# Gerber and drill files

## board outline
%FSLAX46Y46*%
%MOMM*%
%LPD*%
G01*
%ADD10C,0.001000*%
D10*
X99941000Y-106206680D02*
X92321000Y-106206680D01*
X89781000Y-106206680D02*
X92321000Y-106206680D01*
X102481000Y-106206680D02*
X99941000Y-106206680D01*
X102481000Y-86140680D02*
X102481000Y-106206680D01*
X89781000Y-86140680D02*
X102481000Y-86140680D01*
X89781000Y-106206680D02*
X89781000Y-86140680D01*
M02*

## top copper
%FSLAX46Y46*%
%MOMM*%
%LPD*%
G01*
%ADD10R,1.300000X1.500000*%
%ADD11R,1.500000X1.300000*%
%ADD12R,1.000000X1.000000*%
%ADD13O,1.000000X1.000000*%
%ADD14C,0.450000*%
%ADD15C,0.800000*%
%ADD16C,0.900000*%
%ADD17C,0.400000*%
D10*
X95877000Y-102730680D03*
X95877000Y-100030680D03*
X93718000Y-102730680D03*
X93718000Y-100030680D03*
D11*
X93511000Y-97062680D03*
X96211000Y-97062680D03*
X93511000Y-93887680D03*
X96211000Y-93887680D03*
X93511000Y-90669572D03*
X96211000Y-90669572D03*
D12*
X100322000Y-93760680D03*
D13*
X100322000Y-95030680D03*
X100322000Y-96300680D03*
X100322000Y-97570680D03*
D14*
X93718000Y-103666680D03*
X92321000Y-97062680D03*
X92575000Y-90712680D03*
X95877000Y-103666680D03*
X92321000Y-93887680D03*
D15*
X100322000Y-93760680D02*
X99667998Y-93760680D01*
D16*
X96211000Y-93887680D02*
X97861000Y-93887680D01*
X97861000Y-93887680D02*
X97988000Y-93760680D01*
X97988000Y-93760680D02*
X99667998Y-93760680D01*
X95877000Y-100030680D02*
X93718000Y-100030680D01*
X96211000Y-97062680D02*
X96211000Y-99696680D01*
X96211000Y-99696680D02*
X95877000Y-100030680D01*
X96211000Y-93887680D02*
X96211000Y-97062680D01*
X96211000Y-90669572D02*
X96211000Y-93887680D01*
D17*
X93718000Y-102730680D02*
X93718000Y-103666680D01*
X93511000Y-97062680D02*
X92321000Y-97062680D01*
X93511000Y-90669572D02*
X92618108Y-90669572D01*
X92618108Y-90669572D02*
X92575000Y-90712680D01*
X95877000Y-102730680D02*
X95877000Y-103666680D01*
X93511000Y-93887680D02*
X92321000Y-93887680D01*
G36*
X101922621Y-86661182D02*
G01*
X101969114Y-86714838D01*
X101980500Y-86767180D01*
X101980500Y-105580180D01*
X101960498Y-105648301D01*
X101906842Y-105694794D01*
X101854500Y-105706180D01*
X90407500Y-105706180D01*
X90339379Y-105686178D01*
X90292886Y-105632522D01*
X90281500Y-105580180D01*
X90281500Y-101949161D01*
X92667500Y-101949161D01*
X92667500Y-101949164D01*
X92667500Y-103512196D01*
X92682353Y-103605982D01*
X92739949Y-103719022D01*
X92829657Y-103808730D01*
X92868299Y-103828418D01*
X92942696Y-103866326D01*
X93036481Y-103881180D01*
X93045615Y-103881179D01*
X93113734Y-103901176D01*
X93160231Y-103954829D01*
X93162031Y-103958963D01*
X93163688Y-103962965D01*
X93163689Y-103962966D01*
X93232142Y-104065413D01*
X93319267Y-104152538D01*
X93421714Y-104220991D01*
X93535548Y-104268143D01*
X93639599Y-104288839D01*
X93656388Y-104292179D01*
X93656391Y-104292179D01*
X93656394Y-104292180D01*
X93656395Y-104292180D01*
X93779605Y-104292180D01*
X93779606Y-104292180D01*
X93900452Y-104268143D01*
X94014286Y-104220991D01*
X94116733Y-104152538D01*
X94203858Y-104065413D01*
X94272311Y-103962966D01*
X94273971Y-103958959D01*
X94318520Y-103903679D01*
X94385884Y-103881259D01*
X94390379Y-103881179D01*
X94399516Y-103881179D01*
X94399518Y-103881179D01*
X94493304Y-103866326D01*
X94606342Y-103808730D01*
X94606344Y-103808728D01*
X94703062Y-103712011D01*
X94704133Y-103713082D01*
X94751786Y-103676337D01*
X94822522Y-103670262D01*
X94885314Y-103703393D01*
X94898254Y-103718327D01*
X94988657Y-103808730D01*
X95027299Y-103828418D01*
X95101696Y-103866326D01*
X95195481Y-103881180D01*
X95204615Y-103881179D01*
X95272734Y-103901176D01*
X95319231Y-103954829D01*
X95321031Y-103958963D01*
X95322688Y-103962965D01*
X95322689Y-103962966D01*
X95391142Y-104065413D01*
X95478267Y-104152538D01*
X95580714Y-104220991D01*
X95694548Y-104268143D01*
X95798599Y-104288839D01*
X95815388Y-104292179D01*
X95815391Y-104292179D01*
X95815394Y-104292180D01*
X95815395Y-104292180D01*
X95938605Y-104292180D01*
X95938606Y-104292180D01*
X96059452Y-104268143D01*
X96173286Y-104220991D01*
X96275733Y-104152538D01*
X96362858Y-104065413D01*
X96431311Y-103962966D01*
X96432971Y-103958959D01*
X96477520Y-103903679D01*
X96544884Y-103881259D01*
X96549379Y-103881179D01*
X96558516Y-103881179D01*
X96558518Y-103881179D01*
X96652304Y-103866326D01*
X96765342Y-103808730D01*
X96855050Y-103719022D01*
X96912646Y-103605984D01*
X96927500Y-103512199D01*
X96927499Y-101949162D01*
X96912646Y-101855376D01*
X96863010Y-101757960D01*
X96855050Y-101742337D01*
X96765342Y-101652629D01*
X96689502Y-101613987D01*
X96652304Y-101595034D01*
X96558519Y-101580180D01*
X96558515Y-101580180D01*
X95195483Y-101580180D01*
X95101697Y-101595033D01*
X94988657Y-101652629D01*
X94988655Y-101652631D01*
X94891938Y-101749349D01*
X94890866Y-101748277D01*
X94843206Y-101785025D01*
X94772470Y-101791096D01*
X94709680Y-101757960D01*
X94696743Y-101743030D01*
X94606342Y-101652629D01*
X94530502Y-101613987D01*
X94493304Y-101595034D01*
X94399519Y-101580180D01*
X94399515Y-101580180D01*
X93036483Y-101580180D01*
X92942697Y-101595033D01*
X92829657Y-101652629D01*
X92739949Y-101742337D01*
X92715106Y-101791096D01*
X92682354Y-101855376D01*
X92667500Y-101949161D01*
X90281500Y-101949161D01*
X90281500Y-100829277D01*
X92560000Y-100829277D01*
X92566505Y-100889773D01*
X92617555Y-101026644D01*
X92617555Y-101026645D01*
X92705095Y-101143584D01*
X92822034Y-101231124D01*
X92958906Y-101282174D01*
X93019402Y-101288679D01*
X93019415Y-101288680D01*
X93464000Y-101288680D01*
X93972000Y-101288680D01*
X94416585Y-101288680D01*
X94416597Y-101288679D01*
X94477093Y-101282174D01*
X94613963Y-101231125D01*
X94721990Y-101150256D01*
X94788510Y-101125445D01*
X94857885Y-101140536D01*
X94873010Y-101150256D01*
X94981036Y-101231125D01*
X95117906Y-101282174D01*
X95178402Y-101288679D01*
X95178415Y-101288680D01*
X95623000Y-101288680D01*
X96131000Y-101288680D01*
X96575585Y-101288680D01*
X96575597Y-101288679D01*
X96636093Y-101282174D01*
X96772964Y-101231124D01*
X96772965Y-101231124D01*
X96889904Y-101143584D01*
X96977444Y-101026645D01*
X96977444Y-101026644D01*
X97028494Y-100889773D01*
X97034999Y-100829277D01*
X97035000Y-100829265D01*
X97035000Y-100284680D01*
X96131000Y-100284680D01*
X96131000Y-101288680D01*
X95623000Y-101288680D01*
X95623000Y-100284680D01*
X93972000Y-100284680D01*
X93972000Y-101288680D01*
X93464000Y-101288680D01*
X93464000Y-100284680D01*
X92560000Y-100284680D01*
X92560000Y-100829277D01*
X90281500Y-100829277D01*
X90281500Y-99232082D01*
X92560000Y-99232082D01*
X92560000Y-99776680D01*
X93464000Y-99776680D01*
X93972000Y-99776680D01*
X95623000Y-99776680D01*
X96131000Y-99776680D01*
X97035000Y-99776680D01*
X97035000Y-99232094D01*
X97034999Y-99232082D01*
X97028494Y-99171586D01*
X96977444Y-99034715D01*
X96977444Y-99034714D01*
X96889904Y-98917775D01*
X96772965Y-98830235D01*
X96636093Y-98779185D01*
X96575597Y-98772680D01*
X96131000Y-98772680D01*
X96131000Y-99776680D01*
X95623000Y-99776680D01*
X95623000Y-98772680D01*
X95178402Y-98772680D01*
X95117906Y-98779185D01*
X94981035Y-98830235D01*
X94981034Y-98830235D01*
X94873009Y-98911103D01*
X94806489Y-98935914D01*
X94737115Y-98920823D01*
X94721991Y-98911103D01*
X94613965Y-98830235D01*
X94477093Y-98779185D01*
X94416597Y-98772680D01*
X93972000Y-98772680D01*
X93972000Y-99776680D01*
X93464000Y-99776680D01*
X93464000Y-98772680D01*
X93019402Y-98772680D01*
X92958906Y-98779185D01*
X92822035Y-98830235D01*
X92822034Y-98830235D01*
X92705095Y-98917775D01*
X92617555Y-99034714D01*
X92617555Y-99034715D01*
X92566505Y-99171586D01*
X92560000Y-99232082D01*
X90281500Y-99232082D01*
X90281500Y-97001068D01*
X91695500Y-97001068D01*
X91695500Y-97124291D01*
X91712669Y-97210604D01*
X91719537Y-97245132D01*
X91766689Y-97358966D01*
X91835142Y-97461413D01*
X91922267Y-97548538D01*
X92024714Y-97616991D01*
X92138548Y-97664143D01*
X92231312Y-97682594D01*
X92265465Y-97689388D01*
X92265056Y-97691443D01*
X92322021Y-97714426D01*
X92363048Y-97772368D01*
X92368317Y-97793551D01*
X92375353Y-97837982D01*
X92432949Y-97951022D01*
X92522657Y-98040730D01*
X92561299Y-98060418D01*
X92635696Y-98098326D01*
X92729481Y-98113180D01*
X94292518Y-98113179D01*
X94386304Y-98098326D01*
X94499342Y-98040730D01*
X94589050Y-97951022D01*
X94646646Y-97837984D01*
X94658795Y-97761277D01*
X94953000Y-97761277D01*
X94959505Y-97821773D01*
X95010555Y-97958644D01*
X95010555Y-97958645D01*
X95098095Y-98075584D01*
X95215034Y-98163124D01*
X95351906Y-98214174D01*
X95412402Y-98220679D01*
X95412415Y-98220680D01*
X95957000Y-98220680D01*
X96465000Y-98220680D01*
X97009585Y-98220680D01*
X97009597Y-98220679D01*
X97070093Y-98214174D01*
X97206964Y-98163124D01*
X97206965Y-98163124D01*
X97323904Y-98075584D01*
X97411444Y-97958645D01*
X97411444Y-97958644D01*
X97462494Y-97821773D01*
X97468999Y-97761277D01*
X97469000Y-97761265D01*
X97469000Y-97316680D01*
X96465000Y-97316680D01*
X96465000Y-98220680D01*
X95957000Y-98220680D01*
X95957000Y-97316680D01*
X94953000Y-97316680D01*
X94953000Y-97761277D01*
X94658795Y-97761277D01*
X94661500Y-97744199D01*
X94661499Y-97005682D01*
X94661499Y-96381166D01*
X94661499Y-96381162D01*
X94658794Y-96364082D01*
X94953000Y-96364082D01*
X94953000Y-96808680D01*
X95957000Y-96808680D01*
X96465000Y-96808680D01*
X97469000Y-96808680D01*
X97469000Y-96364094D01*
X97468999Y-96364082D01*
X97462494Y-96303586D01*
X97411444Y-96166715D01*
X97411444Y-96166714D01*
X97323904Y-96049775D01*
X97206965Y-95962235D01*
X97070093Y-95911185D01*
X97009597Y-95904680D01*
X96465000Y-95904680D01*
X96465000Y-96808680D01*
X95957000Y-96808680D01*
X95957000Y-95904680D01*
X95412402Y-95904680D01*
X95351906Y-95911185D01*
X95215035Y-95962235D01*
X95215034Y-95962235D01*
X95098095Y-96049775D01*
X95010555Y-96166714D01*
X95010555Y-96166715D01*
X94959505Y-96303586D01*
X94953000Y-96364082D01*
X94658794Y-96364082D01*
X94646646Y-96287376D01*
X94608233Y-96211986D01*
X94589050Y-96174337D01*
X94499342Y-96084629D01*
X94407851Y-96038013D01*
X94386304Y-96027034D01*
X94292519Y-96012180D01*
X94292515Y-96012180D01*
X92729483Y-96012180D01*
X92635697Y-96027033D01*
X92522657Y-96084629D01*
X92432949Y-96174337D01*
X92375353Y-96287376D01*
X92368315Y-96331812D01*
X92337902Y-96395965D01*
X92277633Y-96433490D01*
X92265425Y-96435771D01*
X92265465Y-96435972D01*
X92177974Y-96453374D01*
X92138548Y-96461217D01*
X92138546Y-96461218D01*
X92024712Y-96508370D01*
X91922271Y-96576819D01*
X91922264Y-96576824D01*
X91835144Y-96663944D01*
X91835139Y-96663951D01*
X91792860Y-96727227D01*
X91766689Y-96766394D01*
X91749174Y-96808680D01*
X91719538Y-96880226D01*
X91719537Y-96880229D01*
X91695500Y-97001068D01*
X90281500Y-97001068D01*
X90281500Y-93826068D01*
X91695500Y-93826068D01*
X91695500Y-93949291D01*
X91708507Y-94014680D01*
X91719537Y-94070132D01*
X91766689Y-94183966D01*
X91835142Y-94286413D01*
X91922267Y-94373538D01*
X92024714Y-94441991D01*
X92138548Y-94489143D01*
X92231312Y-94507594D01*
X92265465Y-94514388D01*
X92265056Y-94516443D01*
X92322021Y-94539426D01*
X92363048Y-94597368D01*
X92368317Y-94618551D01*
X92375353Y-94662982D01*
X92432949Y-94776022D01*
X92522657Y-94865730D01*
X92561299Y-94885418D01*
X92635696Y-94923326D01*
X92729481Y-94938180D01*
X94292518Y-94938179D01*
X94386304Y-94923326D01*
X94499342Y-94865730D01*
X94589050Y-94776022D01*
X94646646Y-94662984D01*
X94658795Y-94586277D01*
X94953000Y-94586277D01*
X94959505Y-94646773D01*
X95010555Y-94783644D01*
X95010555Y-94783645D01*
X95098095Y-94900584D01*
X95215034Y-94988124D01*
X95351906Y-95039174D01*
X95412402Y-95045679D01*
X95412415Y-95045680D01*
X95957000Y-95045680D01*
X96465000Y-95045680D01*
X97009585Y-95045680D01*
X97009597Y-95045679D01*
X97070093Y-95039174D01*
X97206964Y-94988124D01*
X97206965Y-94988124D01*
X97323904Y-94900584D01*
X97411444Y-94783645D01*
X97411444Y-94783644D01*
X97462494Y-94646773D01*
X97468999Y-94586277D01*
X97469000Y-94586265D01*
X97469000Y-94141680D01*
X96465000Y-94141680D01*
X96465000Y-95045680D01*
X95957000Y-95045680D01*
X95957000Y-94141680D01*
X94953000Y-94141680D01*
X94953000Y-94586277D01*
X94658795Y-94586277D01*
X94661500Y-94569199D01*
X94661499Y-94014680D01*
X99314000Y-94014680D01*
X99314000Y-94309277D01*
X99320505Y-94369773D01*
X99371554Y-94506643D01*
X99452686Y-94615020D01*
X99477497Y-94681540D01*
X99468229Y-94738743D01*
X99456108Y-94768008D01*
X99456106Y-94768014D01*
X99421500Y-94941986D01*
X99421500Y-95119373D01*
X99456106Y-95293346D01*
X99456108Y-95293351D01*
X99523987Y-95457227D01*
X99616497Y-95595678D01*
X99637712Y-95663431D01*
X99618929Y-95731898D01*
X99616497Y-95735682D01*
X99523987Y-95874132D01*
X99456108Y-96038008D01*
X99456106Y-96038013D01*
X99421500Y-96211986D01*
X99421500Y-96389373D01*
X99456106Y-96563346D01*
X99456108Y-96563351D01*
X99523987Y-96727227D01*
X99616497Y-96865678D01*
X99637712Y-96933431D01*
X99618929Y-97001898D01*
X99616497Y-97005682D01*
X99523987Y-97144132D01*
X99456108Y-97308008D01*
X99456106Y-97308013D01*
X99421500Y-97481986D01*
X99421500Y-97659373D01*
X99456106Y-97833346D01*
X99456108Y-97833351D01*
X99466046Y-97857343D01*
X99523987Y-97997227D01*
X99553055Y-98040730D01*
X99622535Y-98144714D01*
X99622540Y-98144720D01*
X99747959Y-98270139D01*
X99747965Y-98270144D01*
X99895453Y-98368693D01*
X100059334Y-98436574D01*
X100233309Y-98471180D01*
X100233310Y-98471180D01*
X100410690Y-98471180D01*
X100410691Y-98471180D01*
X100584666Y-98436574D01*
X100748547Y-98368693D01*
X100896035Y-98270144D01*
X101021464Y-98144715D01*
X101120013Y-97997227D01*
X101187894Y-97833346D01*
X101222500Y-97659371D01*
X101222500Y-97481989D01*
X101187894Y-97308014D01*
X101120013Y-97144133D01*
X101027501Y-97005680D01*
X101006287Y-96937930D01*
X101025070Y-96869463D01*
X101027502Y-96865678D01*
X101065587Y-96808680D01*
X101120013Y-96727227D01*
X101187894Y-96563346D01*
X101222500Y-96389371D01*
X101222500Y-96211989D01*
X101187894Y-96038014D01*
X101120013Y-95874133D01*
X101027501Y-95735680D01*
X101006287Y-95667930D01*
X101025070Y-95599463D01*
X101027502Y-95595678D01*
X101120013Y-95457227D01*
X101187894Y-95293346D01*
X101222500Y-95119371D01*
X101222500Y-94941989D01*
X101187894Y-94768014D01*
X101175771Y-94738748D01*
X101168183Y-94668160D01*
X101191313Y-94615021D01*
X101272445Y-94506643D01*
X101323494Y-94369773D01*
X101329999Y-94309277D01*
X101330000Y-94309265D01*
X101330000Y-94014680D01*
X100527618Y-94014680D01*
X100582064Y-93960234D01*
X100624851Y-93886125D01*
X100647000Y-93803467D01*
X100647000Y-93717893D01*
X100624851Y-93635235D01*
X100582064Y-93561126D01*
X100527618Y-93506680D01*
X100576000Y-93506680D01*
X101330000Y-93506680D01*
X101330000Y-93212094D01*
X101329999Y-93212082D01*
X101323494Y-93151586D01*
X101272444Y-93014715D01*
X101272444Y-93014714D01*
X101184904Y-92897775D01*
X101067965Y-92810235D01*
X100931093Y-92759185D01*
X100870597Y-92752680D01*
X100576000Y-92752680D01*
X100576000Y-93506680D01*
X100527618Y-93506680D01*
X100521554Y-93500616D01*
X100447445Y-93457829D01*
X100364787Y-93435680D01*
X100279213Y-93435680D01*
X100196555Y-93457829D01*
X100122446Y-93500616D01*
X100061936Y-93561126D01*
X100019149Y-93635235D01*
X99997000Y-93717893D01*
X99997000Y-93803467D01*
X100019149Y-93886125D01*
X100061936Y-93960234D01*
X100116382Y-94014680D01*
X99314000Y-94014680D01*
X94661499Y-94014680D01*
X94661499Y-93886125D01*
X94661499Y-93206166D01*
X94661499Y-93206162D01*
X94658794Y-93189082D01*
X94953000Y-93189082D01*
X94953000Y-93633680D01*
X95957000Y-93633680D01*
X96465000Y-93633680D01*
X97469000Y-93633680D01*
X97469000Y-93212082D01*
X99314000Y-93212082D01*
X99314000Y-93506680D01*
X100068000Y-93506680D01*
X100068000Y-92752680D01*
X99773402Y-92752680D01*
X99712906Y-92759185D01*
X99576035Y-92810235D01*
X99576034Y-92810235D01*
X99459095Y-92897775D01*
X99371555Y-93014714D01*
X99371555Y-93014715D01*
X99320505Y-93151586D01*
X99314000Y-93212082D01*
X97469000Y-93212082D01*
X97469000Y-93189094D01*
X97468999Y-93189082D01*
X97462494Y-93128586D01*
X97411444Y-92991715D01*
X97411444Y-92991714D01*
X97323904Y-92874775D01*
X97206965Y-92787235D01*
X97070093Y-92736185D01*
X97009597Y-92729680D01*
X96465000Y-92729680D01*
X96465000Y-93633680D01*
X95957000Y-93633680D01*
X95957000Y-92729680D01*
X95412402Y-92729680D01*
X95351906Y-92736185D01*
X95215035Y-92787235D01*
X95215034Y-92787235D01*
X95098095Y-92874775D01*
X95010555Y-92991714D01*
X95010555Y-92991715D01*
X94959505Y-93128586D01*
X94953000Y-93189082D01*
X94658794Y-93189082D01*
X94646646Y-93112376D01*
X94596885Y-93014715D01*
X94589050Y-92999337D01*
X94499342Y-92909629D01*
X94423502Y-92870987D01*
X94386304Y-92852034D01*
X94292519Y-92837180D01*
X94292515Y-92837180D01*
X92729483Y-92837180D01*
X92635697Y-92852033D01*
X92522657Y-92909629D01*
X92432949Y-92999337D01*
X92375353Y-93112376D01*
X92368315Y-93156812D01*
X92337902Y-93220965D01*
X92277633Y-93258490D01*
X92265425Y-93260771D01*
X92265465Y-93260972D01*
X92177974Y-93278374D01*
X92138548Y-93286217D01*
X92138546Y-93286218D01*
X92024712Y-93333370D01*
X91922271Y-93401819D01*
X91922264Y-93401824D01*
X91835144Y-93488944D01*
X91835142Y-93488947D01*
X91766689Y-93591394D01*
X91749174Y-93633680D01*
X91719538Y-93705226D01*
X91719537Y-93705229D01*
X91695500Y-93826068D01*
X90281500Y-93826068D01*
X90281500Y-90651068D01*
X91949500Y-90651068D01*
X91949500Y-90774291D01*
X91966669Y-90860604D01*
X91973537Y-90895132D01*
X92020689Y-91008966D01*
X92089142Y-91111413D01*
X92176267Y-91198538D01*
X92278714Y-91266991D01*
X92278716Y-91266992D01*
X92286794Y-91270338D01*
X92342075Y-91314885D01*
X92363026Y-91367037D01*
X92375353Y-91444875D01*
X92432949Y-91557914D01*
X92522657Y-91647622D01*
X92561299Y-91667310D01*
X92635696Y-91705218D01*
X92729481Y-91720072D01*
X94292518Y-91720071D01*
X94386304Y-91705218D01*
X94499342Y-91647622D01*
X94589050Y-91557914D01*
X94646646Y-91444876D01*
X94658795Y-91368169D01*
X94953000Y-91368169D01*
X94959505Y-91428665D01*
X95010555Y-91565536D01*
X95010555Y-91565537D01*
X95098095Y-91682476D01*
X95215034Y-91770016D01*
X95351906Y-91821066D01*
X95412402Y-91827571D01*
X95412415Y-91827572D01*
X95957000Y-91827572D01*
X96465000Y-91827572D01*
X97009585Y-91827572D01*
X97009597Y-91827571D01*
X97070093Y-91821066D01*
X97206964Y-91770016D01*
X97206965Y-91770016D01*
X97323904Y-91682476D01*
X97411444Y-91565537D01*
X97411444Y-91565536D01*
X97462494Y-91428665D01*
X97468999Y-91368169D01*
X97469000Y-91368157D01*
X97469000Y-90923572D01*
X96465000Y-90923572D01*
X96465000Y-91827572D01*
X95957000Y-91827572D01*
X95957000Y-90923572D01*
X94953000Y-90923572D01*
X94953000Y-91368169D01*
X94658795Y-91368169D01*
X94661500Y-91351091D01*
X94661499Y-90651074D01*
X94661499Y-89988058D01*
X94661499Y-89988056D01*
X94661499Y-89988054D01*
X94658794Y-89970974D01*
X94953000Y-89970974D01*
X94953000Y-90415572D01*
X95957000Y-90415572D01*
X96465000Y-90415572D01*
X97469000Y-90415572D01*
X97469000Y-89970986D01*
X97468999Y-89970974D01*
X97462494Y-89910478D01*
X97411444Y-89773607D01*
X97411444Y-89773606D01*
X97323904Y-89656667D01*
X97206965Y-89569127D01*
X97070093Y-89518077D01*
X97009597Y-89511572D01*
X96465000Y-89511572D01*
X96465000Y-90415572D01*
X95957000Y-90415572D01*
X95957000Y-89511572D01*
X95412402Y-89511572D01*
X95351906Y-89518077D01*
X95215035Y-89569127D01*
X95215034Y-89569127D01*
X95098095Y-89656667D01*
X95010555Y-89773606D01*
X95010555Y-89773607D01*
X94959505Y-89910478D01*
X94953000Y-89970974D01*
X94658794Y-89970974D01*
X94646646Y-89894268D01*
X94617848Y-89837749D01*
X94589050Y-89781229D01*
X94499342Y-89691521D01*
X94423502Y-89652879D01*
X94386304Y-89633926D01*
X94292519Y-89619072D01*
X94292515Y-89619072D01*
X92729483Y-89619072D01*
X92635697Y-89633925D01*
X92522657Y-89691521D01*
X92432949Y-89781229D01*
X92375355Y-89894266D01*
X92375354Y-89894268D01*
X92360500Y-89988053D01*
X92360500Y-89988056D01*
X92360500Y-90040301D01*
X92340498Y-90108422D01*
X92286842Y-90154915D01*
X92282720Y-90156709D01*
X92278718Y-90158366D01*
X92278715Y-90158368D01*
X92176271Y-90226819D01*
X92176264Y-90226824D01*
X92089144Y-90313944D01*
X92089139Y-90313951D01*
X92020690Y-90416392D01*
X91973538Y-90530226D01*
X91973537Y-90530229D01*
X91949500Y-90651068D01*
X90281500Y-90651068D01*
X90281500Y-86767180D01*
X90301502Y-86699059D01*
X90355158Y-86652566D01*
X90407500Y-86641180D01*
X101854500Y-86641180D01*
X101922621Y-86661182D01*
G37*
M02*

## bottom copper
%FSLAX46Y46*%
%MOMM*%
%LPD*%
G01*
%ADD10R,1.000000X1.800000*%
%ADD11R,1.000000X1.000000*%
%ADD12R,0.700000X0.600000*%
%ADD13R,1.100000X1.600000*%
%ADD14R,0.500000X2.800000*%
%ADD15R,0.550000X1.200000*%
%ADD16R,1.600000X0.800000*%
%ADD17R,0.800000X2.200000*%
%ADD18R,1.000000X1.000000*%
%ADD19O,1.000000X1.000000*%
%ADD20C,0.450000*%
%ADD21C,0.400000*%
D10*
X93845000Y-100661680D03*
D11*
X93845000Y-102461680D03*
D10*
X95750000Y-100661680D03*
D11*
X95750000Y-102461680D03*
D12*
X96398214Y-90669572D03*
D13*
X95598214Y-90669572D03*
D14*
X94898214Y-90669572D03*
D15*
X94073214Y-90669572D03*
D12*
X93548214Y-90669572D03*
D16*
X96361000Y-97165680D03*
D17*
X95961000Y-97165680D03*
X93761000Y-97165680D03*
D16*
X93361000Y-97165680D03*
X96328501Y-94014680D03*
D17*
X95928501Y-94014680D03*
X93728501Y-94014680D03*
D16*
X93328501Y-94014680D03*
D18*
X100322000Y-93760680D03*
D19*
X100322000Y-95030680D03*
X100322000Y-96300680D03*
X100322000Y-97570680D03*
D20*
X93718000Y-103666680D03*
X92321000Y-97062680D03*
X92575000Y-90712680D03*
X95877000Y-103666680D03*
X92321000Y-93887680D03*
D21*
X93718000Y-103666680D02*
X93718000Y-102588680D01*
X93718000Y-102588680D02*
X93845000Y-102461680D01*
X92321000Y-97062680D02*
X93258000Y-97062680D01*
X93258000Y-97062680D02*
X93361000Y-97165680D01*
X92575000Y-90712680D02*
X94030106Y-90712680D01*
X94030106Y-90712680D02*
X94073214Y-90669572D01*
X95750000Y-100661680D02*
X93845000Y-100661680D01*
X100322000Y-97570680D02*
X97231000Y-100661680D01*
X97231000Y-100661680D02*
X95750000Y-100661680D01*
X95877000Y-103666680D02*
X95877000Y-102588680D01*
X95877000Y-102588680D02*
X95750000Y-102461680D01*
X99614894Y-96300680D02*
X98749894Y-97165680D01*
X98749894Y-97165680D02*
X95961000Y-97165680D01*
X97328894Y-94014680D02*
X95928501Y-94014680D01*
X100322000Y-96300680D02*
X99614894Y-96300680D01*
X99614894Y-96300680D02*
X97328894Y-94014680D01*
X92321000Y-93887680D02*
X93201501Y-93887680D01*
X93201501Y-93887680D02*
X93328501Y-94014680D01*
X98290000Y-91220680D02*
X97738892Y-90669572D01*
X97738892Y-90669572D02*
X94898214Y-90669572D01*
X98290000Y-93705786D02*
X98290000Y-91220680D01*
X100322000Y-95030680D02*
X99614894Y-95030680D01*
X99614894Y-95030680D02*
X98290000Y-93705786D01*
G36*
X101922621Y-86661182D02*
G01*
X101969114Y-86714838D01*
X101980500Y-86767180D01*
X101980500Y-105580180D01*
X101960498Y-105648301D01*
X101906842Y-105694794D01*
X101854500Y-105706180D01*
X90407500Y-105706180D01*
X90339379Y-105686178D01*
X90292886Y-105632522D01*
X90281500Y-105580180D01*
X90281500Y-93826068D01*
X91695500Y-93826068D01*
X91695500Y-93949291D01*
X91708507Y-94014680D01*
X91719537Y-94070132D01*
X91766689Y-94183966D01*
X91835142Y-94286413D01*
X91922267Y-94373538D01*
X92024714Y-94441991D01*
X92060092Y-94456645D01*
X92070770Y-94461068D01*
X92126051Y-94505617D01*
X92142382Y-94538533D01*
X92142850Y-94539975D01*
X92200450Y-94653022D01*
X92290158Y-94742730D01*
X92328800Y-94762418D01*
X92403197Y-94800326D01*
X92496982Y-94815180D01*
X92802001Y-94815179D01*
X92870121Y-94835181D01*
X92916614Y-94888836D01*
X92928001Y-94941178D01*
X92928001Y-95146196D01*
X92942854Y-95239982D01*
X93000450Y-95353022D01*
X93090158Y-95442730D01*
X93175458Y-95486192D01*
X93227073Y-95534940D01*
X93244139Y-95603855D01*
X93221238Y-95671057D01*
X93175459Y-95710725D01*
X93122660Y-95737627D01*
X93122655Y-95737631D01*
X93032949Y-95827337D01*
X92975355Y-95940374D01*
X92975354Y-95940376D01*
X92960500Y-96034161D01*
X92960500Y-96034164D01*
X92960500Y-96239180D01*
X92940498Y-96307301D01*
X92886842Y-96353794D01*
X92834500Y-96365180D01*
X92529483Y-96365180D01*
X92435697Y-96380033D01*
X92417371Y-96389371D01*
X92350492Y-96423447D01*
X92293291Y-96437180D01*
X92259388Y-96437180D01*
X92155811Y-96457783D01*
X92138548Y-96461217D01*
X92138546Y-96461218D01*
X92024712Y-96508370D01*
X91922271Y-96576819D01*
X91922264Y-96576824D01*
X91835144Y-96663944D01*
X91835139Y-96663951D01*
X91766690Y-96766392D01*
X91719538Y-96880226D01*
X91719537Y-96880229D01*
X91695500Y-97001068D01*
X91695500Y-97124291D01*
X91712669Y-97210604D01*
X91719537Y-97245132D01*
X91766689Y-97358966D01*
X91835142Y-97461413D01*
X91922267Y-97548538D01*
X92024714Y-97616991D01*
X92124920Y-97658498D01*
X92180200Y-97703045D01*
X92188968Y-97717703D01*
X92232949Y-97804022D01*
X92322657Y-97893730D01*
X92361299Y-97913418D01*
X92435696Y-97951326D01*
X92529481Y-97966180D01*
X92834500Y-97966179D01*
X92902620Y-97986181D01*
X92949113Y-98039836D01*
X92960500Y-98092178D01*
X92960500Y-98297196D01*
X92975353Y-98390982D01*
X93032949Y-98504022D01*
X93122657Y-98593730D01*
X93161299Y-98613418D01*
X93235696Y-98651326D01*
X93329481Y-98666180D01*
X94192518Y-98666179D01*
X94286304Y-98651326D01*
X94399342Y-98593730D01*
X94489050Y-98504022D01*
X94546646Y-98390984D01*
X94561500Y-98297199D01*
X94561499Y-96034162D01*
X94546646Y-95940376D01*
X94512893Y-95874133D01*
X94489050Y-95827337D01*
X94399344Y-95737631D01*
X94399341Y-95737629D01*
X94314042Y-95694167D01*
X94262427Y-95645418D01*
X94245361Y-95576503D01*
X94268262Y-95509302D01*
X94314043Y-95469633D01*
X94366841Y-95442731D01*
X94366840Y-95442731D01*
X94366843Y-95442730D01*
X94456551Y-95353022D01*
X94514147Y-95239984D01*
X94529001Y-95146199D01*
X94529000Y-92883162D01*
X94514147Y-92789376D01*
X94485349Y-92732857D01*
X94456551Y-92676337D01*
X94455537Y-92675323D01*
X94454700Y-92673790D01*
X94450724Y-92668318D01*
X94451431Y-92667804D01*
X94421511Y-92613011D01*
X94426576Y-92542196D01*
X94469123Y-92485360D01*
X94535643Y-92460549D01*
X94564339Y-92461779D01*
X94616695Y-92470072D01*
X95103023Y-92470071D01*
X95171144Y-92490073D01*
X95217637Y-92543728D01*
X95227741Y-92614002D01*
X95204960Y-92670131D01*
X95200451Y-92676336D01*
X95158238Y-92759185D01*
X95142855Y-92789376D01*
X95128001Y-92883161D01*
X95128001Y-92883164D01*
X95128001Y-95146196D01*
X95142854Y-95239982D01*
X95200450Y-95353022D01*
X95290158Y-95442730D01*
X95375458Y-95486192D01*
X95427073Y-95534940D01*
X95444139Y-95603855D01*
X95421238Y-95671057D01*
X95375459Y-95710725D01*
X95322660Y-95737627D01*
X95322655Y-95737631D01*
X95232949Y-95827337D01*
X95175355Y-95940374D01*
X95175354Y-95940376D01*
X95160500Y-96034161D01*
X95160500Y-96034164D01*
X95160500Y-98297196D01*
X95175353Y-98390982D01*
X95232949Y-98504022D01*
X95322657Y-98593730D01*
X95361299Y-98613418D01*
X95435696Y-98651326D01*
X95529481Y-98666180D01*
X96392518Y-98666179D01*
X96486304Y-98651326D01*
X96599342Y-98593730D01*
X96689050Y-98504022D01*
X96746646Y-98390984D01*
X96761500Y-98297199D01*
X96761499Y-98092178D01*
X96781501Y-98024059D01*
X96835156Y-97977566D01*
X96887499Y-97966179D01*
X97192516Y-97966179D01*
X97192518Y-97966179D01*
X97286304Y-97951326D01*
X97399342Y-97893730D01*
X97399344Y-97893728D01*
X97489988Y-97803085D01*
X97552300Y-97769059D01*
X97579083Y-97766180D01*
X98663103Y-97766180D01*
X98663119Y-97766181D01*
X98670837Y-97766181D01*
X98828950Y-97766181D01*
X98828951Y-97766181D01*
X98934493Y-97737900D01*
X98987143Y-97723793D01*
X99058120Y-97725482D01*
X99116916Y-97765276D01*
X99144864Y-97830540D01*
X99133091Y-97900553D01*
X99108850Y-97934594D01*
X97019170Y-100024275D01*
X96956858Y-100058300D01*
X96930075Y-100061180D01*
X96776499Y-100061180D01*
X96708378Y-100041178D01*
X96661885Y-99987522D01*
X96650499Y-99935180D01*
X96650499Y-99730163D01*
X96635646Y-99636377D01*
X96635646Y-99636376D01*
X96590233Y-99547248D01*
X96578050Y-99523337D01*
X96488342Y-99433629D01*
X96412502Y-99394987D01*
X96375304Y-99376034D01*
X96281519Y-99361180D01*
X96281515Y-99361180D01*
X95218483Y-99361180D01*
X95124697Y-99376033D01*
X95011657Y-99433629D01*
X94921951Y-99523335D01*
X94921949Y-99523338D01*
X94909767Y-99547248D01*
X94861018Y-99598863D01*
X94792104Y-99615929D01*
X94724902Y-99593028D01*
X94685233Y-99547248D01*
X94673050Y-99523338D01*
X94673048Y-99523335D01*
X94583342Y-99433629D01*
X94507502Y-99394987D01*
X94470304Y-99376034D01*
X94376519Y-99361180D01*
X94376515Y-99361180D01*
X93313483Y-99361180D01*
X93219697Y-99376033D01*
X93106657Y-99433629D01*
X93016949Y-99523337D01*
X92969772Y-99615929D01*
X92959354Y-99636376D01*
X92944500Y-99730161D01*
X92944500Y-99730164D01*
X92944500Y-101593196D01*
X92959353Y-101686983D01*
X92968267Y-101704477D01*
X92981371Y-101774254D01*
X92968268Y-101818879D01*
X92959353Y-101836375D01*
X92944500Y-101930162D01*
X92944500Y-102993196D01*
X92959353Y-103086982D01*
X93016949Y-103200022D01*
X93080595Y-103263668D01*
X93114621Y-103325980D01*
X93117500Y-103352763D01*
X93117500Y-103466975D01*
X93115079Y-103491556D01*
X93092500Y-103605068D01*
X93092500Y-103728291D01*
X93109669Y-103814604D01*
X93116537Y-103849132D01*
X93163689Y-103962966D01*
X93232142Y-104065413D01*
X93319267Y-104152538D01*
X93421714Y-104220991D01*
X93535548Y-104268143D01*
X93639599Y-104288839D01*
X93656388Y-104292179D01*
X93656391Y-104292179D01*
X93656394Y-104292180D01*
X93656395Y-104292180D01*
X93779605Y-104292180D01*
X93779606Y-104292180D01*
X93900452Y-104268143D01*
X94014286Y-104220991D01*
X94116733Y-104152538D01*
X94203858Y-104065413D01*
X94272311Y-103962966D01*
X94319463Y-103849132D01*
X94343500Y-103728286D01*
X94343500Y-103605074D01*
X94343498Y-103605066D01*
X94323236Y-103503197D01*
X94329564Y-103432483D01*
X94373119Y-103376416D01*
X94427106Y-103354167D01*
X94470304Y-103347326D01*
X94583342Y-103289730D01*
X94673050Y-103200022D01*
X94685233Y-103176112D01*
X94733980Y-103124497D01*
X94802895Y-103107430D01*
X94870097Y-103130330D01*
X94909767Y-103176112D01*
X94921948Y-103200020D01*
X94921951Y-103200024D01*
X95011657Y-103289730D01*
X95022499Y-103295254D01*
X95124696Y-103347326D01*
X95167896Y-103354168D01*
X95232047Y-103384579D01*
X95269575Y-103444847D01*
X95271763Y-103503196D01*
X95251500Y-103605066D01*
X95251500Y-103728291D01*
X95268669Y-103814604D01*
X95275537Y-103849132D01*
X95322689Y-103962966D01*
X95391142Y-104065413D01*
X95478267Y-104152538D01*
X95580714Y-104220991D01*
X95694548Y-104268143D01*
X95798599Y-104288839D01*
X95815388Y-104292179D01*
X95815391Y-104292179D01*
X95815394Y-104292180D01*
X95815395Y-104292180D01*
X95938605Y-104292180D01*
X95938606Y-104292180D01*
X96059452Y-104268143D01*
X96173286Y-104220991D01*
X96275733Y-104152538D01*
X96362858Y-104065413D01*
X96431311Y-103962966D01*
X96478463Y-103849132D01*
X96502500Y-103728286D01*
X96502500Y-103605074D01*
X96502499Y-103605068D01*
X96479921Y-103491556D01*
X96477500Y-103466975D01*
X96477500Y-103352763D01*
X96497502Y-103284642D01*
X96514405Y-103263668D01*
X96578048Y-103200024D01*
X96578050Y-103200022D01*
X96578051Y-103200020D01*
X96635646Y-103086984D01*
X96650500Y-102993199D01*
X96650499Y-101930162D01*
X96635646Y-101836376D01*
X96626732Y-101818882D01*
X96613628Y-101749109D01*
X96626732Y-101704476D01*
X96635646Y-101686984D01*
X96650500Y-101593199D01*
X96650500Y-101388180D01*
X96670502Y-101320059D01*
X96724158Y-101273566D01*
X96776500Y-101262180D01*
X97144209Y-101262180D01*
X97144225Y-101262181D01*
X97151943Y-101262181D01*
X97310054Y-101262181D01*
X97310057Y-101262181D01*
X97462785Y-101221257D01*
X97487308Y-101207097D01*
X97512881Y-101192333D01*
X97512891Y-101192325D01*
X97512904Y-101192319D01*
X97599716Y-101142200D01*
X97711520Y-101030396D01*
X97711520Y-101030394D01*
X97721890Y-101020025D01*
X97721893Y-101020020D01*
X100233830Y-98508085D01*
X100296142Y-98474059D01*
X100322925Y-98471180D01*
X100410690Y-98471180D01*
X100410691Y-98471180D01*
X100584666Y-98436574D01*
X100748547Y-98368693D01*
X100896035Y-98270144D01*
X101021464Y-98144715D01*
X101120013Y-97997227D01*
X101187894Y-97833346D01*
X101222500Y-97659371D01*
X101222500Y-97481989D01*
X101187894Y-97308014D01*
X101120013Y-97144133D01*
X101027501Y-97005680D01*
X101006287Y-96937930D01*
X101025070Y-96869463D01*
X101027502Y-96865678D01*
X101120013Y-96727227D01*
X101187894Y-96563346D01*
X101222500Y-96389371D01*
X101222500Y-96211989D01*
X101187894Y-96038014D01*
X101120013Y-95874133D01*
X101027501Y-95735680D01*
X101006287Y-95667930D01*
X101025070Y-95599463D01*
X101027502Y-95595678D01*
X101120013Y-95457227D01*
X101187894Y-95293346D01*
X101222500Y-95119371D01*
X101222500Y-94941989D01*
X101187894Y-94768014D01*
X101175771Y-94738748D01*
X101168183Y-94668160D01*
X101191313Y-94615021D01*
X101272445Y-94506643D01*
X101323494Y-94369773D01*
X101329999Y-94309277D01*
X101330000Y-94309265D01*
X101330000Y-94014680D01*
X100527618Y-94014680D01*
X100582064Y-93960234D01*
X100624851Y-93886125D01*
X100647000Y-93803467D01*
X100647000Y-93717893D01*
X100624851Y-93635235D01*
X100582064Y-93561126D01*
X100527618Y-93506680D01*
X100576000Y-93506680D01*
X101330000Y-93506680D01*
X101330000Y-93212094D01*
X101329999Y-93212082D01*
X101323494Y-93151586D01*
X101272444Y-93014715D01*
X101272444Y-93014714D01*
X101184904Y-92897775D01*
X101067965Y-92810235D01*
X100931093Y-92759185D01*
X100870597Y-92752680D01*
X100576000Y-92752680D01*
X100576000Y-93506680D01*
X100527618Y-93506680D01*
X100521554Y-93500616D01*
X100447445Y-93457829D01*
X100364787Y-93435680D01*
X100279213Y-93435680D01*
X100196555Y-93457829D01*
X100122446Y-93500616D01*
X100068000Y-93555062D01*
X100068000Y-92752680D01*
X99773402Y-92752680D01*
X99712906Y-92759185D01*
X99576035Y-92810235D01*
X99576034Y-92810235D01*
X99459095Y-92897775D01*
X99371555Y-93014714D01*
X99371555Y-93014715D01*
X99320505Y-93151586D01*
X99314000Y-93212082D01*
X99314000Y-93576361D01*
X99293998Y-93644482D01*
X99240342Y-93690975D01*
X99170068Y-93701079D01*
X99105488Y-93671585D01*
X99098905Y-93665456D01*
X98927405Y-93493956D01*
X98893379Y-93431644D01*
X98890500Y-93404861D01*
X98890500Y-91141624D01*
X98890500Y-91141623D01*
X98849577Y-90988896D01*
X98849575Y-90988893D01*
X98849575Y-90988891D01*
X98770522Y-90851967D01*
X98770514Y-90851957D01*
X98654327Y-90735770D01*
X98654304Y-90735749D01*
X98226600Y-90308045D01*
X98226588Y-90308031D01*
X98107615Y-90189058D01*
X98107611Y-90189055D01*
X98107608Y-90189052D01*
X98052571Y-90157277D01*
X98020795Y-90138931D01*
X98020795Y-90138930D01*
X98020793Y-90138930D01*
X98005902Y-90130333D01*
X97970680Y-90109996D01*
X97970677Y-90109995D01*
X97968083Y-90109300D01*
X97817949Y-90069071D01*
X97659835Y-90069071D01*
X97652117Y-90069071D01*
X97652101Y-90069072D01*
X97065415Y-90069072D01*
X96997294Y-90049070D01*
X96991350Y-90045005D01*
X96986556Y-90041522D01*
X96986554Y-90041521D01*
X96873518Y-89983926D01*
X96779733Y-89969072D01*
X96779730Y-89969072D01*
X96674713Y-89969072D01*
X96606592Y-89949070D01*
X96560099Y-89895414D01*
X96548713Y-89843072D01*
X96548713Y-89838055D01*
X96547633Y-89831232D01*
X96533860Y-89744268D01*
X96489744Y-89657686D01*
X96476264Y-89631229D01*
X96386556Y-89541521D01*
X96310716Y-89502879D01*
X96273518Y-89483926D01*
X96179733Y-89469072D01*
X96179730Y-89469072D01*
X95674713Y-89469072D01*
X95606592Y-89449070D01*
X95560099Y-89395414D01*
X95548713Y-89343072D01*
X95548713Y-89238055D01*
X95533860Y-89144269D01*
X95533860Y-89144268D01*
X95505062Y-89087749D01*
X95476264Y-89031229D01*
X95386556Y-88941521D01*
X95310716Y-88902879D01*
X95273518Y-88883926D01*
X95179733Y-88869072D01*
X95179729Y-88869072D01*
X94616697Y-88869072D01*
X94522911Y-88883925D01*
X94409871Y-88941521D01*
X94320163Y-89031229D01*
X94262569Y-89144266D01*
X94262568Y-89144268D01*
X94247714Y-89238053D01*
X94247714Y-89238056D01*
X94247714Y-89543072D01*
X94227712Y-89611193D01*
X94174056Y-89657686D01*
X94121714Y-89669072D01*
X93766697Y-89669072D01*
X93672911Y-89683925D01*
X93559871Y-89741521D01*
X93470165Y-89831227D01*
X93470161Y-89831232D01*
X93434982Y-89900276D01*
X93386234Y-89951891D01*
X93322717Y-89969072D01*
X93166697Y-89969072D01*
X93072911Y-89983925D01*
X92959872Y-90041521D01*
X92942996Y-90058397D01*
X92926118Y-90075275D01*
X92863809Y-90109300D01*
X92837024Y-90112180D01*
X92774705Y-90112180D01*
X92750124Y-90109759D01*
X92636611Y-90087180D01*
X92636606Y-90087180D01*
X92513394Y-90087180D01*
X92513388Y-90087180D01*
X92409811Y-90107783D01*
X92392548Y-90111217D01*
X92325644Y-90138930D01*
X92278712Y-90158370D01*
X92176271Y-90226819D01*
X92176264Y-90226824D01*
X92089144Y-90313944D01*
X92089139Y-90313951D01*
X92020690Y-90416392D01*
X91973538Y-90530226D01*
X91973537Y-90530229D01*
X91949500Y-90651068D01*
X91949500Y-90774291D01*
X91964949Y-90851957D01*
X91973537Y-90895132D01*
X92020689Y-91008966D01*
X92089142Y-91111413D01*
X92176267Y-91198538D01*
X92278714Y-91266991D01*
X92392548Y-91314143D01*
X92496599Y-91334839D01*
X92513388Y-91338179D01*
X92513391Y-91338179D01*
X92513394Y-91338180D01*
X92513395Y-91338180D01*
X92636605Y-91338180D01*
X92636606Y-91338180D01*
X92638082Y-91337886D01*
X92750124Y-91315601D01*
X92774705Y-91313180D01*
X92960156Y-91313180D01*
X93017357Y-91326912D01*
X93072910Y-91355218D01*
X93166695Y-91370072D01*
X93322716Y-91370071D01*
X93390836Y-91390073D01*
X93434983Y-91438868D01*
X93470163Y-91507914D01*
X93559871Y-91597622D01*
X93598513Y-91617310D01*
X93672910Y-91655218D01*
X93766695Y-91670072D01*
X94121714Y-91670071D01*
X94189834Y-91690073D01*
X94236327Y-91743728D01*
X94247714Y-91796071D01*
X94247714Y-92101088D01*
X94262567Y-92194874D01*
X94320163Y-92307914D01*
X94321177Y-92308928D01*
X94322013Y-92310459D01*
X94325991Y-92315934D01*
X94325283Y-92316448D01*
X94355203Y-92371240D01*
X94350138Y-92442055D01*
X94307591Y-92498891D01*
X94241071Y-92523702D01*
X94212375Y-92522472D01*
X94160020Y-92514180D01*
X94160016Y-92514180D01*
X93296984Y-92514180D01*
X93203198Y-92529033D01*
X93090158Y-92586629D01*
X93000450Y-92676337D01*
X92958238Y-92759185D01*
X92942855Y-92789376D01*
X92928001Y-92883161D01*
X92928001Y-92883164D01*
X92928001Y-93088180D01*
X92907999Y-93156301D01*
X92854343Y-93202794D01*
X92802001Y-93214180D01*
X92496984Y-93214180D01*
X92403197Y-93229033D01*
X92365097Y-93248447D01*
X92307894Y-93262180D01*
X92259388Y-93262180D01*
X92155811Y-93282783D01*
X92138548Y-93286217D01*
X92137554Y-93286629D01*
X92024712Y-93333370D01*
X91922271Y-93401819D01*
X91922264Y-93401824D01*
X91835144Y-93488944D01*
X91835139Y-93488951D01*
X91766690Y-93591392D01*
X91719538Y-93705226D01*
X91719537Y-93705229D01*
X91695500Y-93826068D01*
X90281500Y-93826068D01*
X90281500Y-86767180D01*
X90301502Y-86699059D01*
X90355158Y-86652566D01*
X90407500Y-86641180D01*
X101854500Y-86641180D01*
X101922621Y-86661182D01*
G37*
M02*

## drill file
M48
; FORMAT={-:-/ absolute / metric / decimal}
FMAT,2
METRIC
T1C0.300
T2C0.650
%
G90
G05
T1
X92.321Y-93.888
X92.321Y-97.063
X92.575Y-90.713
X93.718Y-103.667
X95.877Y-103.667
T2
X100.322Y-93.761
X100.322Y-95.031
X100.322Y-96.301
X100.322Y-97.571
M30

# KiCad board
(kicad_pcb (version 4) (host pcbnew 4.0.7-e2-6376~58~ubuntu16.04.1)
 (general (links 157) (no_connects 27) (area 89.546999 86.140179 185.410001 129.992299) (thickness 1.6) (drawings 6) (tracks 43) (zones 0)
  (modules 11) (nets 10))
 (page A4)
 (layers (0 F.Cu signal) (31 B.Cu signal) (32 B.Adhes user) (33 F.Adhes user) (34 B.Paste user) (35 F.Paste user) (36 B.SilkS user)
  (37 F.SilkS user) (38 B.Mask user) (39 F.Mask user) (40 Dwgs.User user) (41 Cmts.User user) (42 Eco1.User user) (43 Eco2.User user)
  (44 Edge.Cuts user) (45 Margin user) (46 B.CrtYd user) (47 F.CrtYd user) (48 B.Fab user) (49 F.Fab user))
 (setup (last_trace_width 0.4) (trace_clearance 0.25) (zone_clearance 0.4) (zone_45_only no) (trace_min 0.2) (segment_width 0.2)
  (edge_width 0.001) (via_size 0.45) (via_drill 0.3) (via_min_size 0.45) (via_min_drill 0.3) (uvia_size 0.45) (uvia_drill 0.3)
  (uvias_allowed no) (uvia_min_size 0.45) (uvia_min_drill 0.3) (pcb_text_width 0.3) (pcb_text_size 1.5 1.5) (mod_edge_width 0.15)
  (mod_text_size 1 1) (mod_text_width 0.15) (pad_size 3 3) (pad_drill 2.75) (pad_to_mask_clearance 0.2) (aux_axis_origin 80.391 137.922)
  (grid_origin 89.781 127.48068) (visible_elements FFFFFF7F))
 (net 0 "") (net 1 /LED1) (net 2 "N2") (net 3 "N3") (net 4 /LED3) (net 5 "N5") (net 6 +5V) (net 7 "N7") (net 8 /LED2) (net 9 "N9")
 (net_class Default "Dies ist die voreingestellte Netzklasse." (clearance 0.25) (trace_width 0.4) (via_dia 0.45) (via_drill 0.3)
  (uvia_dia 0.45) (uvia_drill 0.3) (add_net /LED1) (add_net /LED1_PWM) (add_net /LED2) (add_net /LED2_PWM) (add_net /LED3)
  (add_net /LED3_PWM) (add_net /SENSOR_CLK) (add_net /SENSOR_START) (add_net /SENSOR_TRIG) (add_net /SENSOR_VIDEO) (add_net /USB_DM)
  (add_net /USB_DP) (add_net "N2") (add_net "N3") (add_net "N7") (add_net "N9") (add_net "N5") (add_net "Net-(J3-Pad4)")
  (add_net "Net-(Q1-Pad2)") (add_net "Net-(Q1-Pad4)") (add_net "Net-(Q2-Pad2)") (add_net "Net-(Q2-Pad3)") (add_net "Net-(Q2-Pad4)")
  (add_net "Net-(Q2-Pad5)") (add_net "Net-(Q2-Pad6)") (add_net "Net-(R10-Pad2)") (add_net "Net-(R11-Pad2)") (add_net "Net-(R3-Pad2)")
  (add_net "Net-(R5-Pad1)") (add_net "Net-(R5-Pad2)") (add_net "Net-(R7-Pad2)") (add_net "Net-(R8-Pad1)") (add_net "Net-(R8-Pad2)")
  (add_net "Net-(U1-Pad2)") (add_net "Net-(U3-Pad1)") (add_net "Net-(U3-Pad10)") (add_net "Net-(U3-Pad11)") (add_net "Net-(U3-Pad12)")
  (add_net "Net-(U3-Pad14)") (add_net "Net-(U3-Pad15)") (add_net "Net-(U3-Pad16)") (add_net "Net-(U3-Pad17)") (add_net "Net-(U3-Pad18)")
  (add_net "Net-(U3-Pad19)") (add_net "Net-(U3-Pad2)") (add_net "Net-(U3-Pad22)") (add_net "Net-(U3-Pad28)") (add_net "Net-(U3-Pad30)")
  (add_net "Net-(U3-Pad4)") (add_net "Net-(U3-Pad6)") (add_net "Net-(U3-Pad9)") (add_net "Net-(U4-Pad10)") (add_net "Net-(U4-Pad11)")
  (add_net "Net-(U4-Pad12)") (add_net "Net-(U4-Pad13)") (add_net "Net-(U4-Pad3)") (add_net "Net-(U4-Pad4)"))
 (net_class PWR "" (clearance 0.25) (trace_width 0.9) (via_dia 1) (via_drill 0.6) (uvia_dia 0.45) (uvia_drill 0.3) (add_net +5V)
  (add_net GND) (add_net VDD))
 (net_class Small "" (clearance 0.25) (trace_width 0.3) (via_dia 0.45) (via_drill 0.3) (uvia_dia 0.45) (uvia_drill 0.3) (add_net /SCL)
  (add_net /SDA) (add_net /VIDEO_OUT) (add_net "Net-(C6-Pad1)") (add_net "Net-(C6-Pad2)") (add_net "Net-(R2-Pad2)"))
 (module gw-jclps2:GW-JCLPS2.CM (layer B.Cu) (at 93.845 101.76168 270)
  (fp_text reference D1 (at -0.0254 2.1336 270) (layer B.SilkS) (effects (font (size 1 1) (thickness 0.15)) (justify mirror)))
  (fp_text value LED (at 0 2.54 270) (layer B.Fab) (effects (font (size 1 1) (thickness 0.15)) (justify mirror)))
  (pad 1 smd rect (at -1.1 0 270) (size 1.8 1) (layers B.Cu B.Paste B.Mask) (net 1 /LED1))
  (pad 2 smd rect (at 0.7 0 270) (size 1 1) (layers B.Cu B.Paste B.Mask) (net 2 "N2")))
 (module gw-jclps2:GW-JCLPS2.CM (layer B.Cu) (at 95.75 101.76168 270)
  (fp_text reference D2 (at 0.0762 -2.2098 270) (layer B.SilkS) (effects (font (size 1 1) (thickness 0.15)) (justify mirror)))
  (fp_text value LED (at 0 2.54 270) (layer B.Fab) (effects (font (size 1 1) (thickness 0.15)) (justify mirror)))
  (pad 1 smd rect (at -1.1 0 270) (size 1.8 1) (layers B.Cu B.Paste B.Mask) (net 1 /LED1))
  (pad 2 smd rect (at 0.7 0 270) (size 1 1) (layers B.Cu B.Paste B.Mask) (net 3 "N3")))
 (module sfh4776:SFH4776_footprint (layer B.Cu) (at 95.148214 90.669572 90)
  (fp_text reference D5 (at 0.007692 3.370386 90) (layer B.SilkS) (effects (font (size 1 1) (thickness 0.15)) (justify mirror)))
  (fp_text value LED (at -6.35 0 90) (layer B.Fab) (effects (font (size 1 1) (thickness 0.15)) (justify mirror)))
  (pad 1 smd rect (at 0 1.25 90) (size 0.6 0.7) (layers B.Cu B.Paste B.Mask) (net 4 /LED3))
  (pad 1 smd rect (at 0 0.45 90) (size 1.6 1.1) (layers B.Cu B.Paste B.Mask) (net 4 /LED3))
  (pad 1 smd rect (at 0 -0.25 90) (size 2.8 0.5) (layers B.Cu B.Paste B.Mask) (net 4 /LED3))
  (pad 2 smd rect (at 0 -1.075 90) (size 1.2 0.55) (layers B.Cu B.Paste B.Mask) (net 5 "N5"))
  (pad 2 smd rect (at 0 -1.6 90) (size 0.6 0.7) (layers B.Cu B.Paste B.Mask) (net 5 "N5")))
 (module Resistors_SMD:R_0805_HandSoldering (layer F.Cu) (at 95.877 101.38068 90)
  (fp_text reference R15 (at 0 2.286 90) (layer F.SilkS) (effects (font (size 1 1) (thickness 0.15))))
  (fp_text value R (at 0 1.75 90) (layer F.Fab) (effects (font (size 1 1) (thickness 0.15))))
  (pad 1 smd rect (at -1.35 0 90) (size 1.5 1.3) (layers F.Cu F.Paste F.Mask) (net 3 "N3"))
  (pad 2 smd rect (at 1.35 0 90) (size 1.5 1.3) (layers F.Cu F.Paste F.Mask) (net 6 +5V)))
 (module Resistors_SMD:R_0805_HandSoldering (layer F.Cu) (at 93.718 101.38068 90)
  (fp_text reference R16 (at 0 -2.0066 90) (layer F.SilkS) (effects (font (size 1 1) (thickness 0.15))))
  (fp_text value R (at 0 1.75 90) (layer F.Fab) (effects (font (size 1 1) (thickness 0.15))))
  (pad 1 smd rect (at -1.35 0 90) (size 1.5 1.3) (layers F.Cu F.Paste F.Mask) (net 2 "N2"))
  (pad 2 smd rect (at 1.35 0 90) (size 1.5 1.3) (layers F.Cu F.Paste F.Mask) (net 6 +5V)))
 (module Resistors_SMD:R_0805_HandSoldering (layer F.Cu) (at 94.861 97.06268)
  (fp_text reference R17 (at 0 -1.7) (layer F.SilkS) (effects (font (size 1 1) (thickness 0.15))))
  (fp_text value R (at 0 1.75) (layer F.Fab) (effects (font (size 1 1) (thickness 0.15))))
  (pad 1 smd rect (at -1.35 0) (size 1.5 1.3) (layers F.Cu F.Paste F.Mask) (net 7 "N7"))
  (pad 2 smd rect (at 1.35 0) (size 1.5 1.3) (layers F.Cu F.Paste F.Mask) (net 6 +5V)))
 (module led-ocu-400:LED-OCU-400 (layer B.Cu) (at 94.861 97.16568)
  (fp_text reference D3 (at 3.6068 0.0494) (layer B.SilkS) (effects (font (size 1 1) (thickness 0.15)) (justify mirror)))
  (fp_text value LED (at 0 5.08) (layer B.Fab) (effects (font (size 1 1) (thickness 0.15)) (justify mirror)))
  (pad 1 smd rect (at 1.5 0) (size 1.6 0.8) (layers B.Cu B.Paste B.Mask) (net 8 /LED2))
  (pad 1 smd rect (at 1.1 0) (size 0.8 2.2) (layers B.Cu B.Paste B.Mask) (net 8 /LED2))
  (pad 2 smd rect (at -1.1 0 180) (size 0.8 2.2) (layers B.Cu B.Paste B.Mask) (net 7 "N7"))
  (pad 2 smd rect (at -1.5 0 180) (size 1.6 0.8) (layers B.Cu B.Paste B.Mask) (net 7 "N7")))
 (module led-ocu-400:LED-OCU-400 (layer B.Cu) (at 94.828501 94.01468)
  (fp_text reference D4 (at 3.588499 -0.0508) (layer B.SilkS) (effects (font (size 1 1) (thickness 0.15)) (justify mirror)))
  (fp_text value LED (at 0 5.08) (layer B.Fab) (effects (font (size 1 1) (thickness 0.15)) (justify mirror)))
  (pad 1 smd rect (at 1.5 0) (size 1.6 0.8) (layers B.Cu B.Paste B.Mask) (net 8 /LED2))
  (pad 1 smd rect (at 1.1 0) (size 0.8 2.2) (layers B.Cu B.Paste B.Mask) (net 8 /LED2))
  (pad 2 smd rect (at -1.1 0 180) (size 0.8 2.2) (layers B.Cu B.Paste B.Mask) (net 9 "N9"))
  (pad 2 smd rect (at -1.5 0 180) (size 1.6 0.8) (layers B.Cu B.Paste B.Mask) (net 9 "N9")))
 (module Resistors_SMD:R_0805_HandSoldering (layer F.Cu) (at 94.861 93.88768)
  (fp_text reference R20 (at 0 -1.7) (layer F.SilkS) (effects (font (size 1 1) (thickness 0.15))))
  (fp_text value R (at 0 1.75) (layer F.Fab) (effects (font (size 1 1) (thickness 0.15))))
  (pad 1 smd rect (at -1.35 0) (size 1.5 1.3) (layers F.Cu F.Paste F.Mask) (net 9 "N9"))
  (pad 2 smd rect (at 1.35 0) (size 1.5 1.3) (layers F.Cu F.Paste F.Mask) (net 6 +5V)))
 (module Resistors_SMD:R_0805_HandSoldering (layer F.Cu) (at 94.861 90.669572)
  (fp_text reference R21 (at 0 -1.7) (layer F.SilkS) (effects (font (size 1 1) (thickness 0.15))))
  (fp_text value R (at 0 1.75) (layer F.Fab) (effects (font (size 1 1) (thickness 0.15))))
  (pad 1 smd rect (at -1.35 0) (size 1.5 1.3) (layers F.Cu F.Paste F.Mask) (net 5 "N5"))
  (pad 2 smd rect (at 1.35 0) (size 1.5 1.3) (layers F.Cu F.Paste F.Mask) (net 6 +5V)))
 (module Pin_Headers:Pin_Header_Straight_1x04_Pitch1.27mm (layer F.Cu) (at 100.322 93.76068)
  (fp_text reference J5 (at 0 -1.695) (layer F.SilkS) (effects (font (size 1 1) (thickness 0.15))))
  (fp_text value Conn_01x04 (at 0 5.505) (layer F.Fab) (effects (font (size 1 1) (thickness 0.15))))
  (pad 1 thru_hole rect (at 0 0) (size 1 1) (drill 0.65) (layers *.Cu *.Mask) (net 6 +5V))
  (pad 2 thru_hole oval (at 0 1.27) (size 1 1) (drill 0.65) (layers *.Cu *.Mask) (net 4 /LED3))
  (pad 3 thru_hole oval (at 0 2.54) (size 1 1) (drill 0.65) (layers *.Cu *.Mask) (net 8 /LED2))
  (pad 4 thru_hole oval (at 0 3.81) (size 1 1) (drill 0.65) (layers *.Cu *.Mask) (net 1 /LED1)))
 (gr_line (start 99.941 106.20668) (end 92.321 106.20668) (layer Edge.Cuts) (width 0.001))
 (gr_line (start 89.781 106.20668) (end 92.321 106.20668) (layer Edge.Cuts) (width 0.001))
 (gr_line (start 102.481 106.20668) (end 99.941 106.20668) (layer Edge.Cuts) (width 0.001))
 (gr_line (start 102.481 86.14068) (end 102.481 106.20668) (layer Edge.Cuts) (width 0.001))
 (gr_line (start 89.781 86.14068) (end 102.481 86.14068) (layer Edge.Cuts) (width 0.001))
 (gr_line (start 89.781 106.20668) (end 89.781 86.14068) (layer Edge.Cuts) (width 0.001))
 (segment (start 100.322 93.76068) (end 99.667998 93.76068) (width 0.8) (layer F.Cu) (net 6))
 (segment (start 96.211 93.88768) (end 97.861 93.88768) (width 0.9) (layer F.Cu) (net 6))
 (segment (start 97.861 93.88768) (end 97.988 93.76068) (width 0.9) (layer F.Cu) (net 6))
 (segment (start 97.988 93.76068) (end 99.667998 93.76068) (width 0.9) (layer F.Cu) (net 6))
 (segment (start 95.877 100.03068) (end 93.718 100.03068) (width 0.9) (layer F.Cu) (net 6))
 (segment (start 96.211 97.06268) (end 96.211 99.69668) (width 0.9) (layer F.Cu) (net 6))
 (segment (start 96.211 99.69668) (end 95.877 100.03068) (width 0.9) (layer F.Cu) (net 6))
 (segment (start 96.211 93.88768) (end 96.211 97.06268) (width 0.9) (layer F.Cu) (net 6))
 (segment (start 96.211 90.669572) (end 96.211 93.88768) (width 0.9) (layer F.Cu) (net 6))
 (segment (start 93.718 103.66668) (end 93.718 102.58868) (width 0.4) (layer B.Cu) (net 2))
 (segment (start 93.718 102.58868) (end 93.845 102.46168) (width 0.4) (layer B.Cu) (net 2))
 (segment (start 93.718 102.73068) (end 93.718 103.66668) (width 0.4) (layer F.Cu) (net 2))
 (via (at 93.718 103.66668) (size 0.45) (drill 0.3) (layers F.Cu B.Cu) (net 2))
 (segment (start 92.321 97.06268) (end 93.258 97.06268) (width 0.4) (layer B.Cu) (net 7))
 (segment (start 93.258 97.06268) (end 93.361 97.16568) (width 0.4) (layer B.Cu) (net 7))
 (segment (start 93.511 97.06268) (end 92.321 97.06268) (width 0.4) (layer F.Cu) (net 7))
 (via (at 92.321 97.06268) (size 0.45) (drill 0.3) (layers F.Cu B.Cu) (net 7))
 (segment (start 92.575 90.71268) (end 94.030106 90.71268) (width 0.4) (layer B.Cu) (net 5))
 (segment (start 94.030106 90.71268) (end 94.073214 90.669572) (width 0.4) (layer B.Cu) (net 5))
 (segment (start 93.511 90.669572) (end 92.618108 90.669572) (width 0.4) (layer F.Cu) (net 5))
 (segment (start 92.618108 90.669572) (end 92.575 90.71268) (width 0.4) (layer F.Cu) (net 5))
 (via (at 92.575 90.71268) (size 0.45) (drill 0.3) (layers F.Cu B.Cu) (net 5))
 (segment (start 95.75 100.66168) (end 93.845 100.66168) (width 0.4) (layer B.Cu) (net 1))
 (segment (start 100.322 97.57068) (end 97.231 100.66168) (width 0.4) (layer B.Cu) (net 1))
 (segment (start 97.231 100.66168) (end 95.75 100.66168) (width 0.4) (layer B.Cu) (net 1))
 (segment (start 95.877 103.66668) (end 95.877 102.58868) (width 0.4) (layer B.Cu) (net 3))
 (segment (start 95.877 102.58868) (end 95.75 102.46168) (width 0.4) (layer B.Cu) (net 3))
 (segment (start 95.877 102.73068) (end 95.877 103.66668) (width 0.4) (layer F.Cu) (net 3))
 (via (at 95.877 103.66668) (size 0.45) (drill 0.3) (layers F.Cu B.Cu) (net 3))
 (segment (start 99.614894 96.30068) (end 98.749894 97.16568) (width 0.4) (layer B.Cu) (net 8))
 (segment (start 98.749894 97.16568) (end 95.961 97.16568) (width 0.4) (layer B.Cu) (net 8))
 (segment (start 97.328894 94.01468) (end 95.928501 94.01468) (width 0.4) (layer B.Cu) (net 8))
 (segment (start 100.322 96.30068) (end 99.614894 96.30068) (width 0.4) (layer B.Cu) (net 8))
 (segment (start 99.614894 96.30068) (end 97.328894 94.01468) (width 0.4) (layer B.Cu) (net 8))
 (segment (start 92.321 93.88768) (end 93.201501 93.88768) (width 0.4) (layer B.Cu) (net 9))
 (segment (start 93.201501 93.88768) (end 93.328501 94.01468) (width 0.4) (layer B.Cu) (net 9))
 (segment (start 93.511 93.88768) (end 92.321 93.88768) (width 0.4) (layer F.Cu) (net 9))
 (via (at 92.321 93.88768) (size 0.45) (drill 0.3) (layers F.Cu B.Cu) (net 9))
 (segment (start 98.29 91.22068) (end 97.738892 90.669572) (width 0.4) (layer B.Cu) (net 4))
 (segment (start 97.738892 90.669572) (end 94.898214 90.669572) (width 0.4) (layer B.Cu) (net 4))
 (segment (start 98.29 93.705786) (end 98.29 91.22068) (width 0.4) (layer B.Cu) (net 4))
 (segment (start 100.322 95.03068) (end 99.614894 95.03068) (width 0.4) (layer B.Cu) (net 4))
 (segment (start 99.614894 95.03068) (end 98.29 93.705786) (width 0.4) (layer B.Cu) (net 4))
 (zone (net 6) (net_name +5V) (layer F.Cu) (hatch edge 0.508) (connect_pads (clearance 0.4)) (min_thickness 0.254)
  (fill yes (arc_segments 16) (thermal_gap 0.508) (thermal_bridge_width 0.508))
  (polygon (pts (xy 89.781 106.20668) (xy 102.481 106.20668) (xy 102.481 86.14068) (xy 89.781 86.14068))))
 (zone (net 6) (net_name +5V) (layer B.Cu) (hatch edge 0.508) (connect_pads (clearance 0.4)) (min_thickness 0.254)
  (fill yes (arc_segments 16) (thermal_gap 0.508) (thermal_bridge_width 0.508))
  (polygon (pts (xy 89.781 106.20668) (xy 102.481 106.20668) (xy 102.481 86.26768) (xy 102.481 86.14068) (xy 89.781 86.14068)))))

